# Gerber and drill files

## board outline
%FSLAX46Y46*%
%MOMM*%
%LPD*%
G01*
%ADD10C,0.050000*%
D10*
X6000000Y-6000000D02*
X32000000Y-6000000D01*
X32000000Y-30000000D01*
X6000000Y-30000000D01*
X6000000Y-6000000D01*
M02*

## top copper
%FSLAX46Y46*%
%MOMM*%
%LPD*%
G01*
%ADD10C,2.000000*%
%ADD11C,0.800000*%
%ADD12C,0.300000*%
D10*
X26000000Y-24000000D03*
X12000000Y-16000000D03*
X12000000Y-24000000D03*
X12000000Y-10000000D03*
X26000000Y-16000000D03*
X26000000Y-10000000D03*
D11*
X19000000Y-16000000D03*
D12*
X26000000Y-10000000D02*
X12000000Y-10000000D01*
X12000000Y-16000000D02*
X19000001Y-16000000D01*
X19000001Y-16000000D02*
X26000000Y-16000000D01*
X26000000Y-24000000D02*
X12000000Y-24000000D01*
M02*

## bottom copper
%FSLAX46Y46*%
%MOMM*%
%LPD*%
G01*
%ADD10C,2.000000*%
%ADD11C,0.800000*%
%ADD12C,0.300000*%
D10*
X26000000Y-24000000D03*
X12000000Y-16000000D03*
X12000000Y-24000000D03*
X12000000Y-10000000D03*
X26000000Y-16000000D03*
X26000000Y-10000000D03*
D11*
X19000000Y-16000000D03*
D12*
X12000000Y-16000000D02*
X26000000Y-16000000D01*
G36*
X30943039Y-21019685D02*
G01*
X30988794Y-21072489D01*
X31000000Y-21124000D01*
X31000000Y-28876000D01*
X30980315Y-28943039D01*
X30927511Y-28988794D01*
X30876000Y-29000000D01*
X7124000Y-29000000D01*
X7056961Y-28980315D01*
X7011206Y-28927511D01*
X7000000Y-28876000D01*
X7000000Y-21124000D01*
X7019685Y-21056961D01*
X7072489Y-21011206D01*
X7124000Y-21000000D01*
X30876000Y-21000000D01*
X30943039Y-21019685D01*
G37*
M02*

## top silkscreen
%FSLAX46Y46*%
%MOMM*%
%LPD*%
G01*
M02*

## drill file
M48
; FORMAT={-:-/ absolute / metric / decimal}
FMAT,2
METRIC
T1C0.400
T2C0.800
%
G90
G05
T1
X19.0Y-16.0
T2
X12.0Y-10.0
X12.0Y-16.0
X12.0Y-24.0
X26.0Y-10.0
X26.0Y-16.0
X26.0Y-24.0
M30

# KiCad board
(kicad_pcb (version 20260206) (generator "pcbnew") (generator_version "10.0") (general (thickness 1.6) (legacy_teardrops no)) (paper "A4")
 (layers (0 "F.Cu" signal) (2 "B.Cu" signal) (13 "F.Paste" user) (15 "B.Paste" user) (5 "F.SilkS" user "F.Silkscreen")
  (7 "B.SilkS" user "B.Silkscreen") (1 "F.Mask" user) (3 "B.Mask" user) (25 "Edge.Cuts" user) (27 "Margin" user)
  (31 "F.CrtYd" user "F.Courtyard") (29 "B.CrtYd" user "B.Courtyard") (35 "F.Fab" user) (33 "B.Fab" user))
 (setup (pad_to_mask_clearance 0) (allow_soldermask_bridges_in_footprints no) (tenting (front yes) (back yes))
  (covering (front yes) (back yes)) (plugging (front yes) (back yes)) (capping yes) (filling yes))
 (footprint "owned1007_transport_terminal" (layer "F.Cu") (at 26 24)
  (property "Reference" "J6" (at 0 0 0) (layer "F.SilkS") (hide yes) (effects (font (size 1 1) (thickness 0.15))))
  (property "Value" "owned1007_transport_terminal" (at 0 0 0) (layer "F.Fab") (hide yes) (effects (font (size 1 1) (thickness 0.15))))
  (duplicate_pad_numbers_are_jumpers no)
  (pad "1" thru_hole circle (at 0 0) (size 2 2) (drill 0.8) (layers "*.Cu" "*.Mask") (remove_unused_layers no) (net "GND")))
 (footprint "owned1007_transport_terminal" (layer "F.Cu") (at 12 16)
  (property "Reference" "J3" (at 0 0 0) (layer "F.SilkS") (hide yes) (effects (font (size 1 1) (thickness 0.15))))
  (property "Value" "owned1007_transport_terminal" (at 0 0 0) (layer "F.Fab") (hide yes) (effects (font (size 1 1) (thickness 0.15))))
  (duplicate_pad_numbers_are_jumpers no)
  (pad "1" thru_hole circle (at 0 0) (size 2 2) (drill 0.8) (layers "*.Cu" "*.Mask") (remove_unused_layers no) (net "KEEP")))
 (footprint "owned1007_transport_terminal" (layer "F.Cu") (at 12 24)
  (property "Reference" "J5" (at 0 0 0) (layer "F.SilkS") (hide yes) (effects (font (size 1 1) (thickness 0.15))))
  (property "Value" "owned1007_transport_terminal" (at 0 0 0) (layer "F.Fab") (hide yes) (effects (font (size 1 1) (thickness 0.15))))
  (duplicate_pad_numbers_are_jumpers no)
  (pad "1" thru_hole circle (at 0 0) (size 2 2) (drill 0.8) (layers "*.Cu" "*.Mask") (remove_unused_layers no) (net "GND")))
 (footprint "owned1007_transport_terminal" (layer "F.Cu") (at 12 10)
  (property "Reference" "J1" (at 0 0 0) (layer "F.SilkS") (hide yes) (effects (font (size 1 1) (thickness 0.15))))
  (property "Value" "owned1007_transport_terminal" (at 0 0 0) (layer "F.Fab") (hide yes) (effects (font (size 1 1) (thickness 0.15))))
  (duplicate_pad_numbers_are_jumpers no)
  (pad "1" thru_hole circle (at 0 0) (size 2 2) (drill 0.8) (layers "*.Cu" "*.Mask") (remove_unused_layers no) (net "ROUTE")))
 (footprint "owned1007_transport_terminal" (layer "F.Cu") (at 26 16)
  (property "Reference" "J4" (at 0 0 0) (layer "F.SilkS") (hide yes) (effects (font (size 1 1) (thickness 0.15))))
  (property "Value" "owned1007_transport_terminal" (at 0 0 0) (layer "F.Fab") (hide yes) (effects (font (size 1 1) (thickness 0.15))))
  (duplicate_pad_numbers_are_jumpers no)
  (pad "1" thru_hole circle (at 0 0) (size 2 2) (drill 0.8) (layers "*.Cu" "*.Mask") (remove_unused_layers no) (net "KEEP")))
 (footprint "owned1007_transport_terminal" (layer "F.Cu") (at 26 10)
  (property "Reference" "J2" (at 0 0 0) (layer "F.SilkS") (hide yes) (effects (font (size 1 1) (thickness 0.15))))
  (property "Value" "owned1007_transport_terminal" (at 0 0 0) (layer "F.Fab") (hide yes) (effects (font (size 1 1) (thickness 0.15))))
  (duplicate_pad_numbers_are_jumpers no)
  (pad "1" thru_hole circle (at 0 0) (size 2 2) (drill 0.8) (layers "*.Cu" "*.Mask") (remove_unused_layers no) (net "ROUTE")))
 (gr_rect (start 6 6) (end 32 30) (stroke (width 0.05) (type default)) (fill no) (layer "Edge.Cuts"))
 (segment (start 26 10) (end 12 10) (width 0.3) (layer "F.Cu") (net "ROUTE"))
 (segment (start 12 16) (end 19.000001 16) (width 0.3) (layer "F.Cu") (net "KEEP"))
 (segment (start 19.000001 16) (end 26 16) (width 0.3) (layer "F.Cu") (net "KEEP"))
 (via (at 19 16) (size 0.8) (drill 0.4) (layers "F.Cu" "B.Cu") (capping yes) (covering (front no) (back no)) (plugging (front no) (back no))
  (filling no) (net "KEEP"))
 (segment (start 12 16) (end 26 16) (width 0.3) (layer "B.Cu") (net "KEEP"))
 (segment (start 26 24) (end 12 24) (width 0.3) (layer "F.Cu") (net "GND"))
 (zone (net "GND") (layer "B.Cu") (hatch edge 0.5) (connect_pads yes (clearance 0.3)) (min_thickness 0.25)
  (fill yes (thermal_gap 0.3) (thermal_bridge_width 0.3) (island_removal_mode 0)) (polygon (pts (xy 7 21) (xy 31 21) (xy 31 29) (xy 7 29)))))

